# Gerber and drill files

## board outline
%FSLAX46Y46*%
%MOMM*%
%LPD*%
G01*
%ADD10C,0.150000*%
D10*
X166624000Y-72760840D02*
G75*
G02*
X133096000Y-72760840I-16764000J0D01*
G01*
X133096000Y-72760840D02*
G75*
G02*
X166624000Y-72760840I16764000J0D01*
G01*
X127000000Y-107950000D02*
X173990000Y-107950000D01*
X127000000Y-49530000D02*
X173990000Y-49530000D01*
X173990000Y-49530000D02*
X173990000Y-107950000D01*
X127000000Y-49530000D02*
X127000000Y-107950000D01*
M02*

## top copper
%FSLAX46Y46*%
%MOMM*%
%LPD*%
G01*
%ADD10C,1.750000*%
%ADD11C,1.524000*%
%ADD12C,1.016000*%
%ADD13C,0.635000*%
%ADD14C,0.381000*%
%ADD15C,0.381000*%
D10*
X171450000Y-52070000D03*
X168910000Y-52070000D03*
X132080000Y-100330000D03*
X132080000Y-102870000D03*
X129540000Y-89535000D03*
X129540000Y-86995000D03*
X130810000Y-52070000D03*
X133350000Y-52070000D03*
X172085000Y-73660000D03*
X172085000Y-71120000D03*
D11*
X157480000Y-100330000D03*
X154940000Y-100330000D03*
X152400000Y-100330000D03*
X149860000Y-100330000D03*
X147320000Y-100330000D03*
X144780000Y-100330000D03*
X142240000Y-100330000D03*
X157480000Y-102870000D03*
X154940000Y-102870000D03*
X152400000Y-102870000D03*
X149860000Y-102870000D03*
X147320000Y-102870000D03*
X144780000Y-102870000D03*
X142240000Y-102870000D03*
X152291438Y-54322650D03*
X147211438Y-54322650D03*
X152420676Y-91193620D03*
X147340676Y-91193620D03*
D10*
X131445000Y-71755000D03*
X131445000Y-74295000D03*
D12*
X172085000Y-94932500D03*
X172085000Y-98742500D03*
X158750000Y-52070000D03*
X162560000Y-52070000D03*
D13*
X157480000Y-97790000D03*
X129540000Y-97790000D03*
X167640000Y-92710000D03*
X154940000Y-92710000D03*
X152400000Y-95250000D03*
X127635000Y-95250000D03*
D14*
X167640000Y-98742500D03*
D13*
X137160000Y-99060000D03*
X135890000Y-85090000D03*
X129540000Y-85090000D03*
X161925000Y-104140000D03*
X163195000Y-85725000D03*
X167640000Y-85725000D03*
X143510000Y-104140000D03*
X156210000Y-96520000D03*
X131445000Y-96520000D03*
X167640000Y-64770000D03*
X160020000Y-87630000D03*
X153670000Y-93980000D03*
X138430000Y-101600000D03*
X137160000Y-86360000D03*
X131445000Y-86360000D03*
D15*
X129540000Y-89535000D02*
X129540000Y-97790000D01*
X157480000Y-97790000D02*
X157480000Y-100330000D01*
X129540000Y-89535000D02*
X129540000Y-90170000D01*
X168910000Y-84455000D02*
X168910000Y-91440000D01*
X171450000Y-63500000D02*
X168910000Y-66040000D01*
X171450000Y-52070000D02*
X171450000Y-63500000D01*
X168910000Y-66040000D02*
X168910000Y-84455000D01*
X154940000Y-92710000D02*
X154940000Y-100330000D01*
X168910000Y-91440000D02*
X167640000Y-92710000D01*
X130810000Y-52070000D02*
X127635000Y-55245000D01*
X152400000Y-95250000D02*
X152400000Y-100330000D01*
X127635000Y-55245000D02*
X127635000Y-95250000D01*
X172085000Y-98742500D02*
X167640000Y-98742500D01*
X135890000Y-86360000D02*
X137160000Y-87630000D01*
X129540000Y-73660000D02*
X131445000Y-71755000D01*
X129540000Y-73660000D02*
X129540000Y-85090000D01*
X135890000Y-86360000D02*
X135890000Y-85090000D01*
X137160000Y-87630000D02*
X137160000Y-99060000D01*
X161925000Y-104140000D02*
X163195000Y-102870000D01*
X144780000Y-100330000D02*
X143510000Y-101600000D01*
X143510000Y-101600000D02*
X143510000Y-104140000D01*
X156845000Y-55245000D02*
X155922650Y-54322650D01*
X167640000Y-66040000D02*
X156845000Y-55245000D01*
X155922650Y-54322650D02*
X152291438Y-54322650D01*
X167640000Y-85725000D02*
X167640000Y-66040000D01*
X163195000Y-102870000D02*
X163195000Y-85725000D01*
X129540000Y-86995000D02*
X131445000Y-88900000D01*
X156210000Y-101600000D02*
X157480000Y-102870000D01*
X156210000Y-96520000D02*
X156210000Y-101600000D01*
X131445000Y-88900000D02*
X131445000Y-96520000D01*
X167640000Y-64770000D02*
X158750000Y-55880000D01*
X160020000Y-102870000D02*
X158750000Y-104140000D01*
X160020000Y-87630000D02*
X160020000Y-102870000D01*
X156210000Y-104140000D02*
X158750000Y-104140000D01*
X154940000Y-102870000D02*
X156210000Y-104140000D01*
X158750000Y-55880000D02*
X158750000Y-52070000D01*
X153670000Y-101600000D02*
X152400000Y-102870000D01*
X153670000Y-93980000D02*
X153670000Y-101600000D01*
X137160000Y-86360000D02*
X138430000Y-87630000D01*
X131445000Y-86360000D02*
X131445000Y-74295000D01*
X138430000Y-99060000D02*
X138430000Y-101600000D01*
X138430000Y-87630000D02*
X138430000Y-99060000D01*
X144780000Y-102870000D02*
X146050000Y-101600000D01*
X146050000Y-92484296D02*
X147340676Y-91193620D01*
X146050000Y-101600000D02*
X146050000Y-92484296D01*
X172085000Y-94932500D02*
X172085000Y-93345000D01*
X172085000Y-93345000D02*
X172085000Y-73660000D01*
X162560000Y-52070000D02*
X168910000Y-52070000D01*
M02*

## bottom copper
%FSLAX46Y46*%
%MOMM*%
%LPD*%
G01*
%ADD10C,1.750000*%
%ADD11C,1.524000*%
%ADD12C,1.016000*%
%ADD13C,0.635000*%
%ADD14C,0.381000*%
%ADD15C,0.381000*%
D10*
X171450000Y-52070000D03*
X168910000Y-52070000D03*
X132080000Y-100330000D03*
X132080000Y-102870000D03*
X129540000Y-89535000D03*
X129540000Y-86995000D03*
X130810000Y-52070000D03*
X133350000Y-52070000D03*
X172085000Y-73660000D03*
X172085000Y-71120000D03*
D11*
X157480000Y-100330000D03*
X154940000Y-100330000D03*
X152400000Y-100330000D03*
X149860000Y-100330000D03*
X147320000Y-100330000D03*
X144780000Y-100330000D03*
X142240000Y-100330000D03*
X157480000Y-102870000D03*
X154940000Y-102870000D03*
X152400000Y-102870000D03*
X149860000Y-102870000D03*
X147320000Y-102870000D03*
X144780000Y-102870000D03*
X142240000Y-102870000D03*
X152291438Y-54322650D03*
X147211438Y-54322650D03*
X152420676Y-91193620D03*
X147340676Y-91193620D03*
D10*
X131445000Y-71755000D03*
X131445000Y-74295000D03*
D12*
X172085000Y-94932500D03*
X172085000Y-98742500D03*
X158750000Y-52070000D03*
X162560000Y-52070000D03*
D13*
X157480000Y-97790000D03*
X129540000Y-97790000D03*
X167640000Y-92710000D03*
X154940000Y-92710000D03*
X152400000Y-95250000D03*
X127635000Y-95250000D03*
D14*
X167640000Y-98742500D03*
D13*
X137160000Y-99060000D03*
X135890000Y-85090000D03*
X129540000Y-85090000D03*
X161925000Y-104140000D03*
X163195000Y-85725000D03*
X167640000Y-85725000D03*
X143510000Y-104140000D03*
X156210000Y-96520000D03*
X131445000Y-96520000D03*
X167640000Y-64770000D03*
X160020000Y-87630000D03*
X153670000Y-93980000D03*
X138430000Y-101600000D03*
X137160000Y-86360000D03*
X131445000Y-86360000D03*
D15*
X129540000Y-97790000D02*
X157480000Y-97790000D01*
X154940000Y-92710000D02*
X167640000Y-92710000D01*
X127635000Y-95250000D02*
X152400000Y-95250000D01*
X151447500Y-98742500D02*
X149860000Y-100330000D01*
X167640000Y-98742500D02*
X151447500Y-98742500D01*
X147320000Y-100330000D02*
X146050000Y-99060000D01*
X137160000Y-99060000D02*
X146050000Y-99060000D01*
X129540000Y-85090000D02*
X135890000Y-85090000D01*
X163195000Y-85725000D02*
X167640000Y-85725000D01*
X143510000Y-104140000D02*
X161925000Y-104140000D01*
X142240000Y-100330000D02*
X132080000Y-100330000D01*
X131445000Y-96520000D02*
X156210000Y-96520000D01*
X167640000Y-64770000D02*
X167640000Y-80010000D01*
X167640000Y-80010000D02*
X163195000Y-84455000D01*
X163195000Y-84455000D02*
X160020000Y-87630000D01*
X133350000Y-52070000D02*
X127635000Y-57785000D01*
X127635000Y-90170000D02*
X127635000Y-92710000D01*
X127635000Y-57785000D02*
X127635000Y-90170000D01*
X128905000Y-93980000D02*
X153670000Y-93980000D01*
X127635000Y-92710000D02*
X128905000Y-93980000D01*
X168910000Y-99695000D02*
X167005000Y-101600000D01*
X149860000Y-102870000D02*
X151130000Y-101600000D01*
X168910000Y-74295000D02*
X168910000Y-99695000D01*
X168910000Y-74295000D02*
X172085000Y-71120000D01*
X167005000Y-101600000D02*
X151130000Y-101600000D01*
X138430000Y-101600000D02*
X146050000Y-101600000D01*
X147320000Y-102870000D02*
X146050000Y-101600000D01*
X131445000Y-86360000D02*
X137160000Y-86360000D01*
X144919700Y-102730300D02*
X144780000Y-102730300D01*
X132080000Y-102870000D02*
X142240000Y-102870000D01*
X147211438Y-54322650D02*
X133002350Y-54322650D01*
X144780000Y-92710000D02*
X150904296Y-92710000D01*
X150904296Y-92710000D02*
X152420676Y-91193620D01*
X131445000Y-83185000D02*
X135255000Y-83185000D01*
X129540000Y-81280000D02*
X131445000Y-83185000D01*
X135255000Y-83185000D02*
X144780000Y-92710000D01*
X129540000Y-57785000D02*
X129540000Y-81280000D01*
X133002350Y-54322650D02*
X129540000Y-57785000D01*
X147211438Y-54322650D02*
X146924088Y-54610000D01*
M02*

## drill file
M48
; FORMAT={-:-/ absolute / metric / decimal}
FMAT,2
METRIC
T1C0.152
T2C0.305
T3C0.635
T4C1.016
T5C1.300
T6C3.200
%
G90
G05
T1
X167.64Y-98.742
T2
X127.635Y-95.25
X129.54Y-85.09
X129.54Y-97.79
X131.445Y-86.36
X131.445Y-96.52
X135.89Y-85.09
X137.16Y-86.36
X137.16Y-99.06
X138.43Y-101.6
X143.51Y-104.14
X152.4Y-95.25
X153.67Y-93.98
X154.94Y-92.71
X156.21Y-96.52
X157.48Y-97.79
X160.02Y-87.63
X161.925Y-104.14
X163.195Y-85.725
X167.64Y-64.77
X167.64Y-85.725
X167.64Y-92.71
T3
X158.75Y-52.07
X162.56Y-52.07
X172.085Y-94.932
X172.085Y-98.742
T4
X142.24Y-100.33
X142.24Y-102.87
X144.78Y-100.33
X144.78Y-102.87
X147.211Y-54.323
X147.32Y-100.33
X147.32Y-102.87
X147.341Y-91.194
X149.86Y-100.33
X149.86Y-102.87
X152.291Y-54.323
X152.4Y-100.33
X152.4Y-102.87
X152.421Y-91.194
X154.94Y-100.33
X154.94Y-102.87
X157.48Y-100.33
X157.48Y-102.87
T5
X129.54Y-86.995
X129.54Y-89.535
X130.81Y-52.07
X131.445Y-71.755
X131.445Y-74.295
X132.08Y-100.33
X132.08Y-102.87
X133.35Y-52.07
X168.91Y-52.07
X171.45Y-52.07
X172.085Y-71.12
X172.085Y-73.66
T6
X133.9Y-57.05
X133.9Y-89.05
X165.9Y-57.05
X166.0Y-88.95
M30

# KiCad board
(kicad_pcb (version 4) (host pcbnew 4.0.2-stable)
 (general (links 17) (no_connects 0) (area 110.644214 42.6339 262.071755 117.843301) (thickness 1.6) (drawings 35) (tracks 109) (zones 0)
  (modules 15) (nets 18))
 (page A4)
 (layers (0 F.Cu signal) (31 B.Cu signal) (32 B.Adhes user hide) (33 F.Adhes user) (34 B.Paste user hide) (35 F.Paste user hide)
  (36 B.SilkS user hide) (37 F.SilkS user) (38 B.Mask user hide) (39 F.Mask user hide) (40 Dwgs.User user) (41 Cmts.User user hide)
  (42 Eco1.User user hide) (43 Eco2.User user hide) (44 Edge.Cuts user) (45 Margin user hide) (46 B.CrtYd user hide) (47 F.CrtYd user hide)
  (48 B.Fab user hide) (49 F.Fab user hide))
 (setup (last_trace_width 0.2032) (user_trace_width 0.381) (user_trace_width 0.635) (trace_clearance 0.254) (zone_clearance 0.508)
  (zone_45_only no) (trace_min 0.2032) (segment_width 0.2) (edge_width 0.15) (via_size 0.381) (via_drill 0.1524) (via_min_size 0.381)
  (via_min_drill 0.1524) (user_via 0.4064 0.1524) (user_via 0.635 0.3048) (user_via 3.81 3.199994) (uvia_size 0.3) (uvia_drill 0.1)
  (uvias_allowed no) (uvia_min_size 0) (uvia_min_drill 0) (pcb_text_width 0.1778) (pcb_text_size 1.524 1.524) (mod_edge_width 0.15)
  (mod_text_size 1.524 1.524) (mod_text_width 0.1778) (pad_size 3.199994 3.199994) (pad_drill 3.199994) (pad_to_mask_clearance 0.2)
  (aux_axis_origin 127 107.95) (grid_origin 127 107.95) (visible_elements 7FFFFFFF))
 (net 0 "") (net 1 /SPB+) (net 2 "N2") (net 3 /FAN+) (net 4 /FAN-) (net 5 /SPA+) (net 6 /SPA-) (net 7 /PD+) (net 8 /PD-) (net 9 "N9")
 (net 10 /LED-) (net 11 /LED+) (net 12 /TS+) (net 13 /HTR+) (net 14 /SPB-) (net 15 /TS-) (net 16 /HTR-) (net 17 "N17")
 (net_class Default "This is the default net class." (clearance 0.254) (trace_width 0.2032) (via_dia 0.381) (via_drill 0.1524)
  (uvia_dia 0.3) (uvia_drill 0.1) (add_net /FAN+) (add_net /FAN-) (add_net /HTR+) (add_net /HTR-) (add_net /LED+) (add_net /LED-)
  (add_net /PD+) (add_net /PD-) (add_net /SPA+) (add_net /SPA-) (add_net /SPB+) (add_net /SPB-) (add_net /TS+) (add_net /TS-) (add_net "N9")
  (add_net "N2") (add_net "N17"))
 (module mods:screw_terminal (layer F.Cu) (at 170.18 52.07 180)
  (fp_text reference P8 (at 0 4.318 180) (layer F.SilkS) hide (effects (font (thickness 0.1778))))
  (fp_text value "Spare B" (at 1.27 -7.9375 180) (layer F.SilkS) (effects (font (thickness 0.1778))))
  (pad 1 thru_hole circle (at -1.27 0 180) (size 1.75 1.75) (drill 1.3) (layers *.Cu *.Mask F.SilkS) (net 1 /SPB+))
  (pad 2 thru_hole circle (at 1.27 0 180) (size 1.75 1.75) (drill 1.3) (layers *.Cu *.Mask F.SilkS) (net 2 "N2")))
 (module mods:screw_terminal (layer F.Cu) (at 132.08 101.6 270)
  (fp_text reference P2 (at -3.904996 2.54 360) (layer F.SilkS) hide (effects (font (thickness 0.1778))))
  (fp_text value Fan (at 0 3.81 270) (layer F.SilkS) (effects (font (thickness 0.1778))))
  (pad 1 thru_hole circle (at -1.27 0 270) (size 1.75 1.75) (drill 1.3) (layers *.Cu *.Mask F.SilkS) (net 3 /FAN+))
  (pad 2 thru_hole circle (at 1.27 0 270) (size 1.75 1.75) (drill 1.3) (layers *.Cu *.Mask F.SilkS) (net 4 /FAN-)))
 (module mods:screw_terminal (layer F.Cu) (at 129.54 88.265 90)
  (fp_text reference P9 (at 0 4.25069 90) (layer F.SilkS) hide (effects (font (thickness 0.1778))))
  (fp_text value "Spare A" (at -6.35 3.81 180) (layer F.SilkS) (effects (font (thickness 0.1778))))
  (pad 1 thru_hole circle (at -1.27 0 90) (size 1.75 1.75) (drill 1.3) (layers *.Cu *.Mask F.SilkS) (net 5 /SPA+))
  (pad 2 thru_hole circle (at 1.27 0 90) (size 1.75 1.75) (drill 1.3) (layers *.Cu *.Mask F.SilkS) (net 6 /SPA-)))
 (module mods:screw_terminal (layer F.Cu) (at 132.08 52.07)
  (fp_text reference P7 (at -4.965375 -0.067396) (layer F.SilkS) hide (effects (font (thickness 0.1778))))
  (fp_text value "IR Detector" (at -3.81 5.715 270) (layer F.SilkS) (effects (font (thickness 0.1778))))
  (pad 1 thru_hole circle (at -1.27 0) (size 1.75 1.75) (drill 1.3) (layers *.Cu *.Mask F.SilkS) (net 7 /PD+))
  (pad 2 thru_hole circle (at 1.27 0) (size 1.75 1.75) (drill 1.3) (layers *.Cu *.Mask F.SilkS) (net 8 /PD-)))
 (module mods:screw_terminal (layer F.Cu) (at 172.085 72.39 90)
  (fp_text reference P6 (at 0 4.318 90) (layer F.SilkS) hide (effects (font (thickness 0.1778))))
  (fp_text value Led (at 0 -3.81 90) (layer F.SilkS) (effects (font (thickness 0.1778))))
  (pad 1 thru_hole circle (at -1.27 0 90) (size 1.75 1.75) (drill 1.3) (layers *.Cu *.Mask F.SilkS) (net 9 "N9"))
  (pad 2 thru_hole circle (at 1.27 0 90) (size 1.75 1.75) (drill 1.3) (layers *.Cu *.Mask F.SilkS) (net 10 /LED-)))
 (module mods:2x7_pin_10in (layer F.Cu) (at 149.86 101.6 180)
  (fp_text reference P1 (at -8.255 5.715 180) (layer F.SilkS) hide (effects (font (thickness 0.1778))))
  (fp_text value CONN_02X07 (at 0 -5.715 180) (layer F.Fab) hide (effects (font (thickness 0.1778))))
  (pad 1 thru_hole circle (at -7.62 1.27 180) (size 1.524 1.524) (drill 1.016) (layers *.Cu *.Mask F.SilkS) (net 5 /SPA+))
  (pad 3 thru_hole circle (at -5.08 1.27 180) (size 1.524 1.524) (drill 1.016) (layers *.Cu *.Mask F.SilkS) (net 1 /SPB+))
  (pad 5 thru_hole circle (at -2.54 1.27 180) (size 1.524 1.524) (drill 1.016) (layers *.Cu *.Mask F.SilkS) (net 7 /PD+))
  (pad 7 thru_hole circle (at 0 1.27 180) (size 1.524 1.524) (drill 1.016) (layers *.Cu *.Mask F.SilkS) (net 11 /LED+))
  (pad 9 thru_hole circle (at 2.54 1.27 180) (size 1.524 1.524) (drill 1.016) (layers *.Cu *.Mask F.SilkS) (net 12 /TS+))
  (pad 11 thru_hole circle (at 5.08 1.27 180) (size 1.524 1.524) (drill 1.016) (layers *.Cu *.Mask F.SilkS) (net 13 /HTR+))
  (pad 13 thru_hole circle (at 7.62 1.27 180) (size 1.524 1.524) (drill 1.016) (layers *.Cu *.Mask F.SilkS) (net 3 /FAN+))
  (pad 2 thru_hole circle (at -7.62 -1.27 180) (size 1.524 1.524) (drill 1.016) (layers *.Cu *.Mask F.SilkS) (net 6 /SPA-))
  (pad 4 thru_hole circle (at -5.08 -1.27 180) (size 1.524 1.524) (drill 1.016) (layers *.Cu *.Mask F.SilkS) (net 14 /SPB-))
  (pad 6 thru_hole circle (at -2.54 -1.27 180) (size 1.524 1.524) (drill 1.016) (layers *.Cu *.Mask F.SilkS) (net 8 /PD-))
  (pad 8 thru_hole circle (at 0 -1.27 180) (size 1.524 1.524) (drill 1.016) (layers *.Cu *.Mask F.SilkS) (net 10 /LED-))
  (pad 10 thru_hole circle (at 2.54 -1.27 180) (size 1.524 1.524) (drill 1.016) (layers *.Cu *.Mask F.SilkS) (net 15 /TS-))
  (pad 12 thru_hole circle (at 5.08 -1.27 180) (size 1.524 1.524) (drill 1.016) (layers *.Cu *.Mask F.SilkS) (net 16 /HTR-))
  (pad 14 thru_hole circle (at 7.62 -1.27 180) (size 1.524 1.524) (drill 1.016) (layers *.Cu *.Mask F.SilkS) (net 4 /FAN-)))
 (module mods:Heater (layer F.Cu) (at 149.751438 54.32265 180)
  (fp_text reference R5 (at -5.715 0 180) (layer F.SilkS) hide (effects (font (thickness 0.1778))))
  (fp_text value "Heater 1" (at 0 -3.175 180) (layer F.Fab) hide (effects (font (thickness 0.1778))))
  (pad 1 thru_hole circle (at -2.54 0 180) (size 1.524 1.524) (drill 1.016) (layers *.Cu *.Mask F.SilkS) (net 13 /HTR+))
  (pad 2 thru_hole circle (at 2.54 0 180) (size 1.524 1.524) (drill 1.016) (layers *.Cu *.Mask F.SilkS) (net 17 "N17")))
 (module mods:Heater (layer F.Cu) (at 149.880676 91.19362 180)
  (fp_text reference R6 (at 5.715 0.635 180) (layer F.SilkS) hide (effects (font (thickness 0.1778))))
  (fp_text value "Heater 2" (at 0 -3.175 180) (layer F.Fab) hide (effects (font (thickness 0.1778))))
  (pad 1 thru_hole circle (at -2.54 0 180) (size 1.524 1.524) (drill 1.016) (layers *.Cu *.Mask F.SilkS) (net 17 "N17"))
  (pad 2 thru_hole circle (at 2.54 0 180) (size 1.524 1.524) (drill 1.016) (layers *.Cu *.Mask F.SilkS) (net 16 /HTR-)))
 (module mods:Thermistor (layer F.Cu) (at 131.445 73.025 270)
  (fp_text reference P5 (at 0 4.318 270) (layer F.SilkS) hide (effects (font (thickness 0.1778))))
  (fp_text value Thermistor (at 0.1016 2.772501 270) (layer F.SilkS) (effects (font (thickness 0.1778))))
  (pad 1 thru_hole circle (at -1.27 0 270) (size 1.75 1.75) (drill 1.3) (layers *.Cu *.Mask F.SilkS) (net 12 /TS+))
  (pad 2 thru_hole circle (at 1.27 0 270) (size 1.75 1.75) (drill 1.3) (layers *.Cu *.Mask F.SilkS) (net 15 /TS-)))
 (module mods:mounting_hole (layer F.Cu) (at 165.9 57.049924)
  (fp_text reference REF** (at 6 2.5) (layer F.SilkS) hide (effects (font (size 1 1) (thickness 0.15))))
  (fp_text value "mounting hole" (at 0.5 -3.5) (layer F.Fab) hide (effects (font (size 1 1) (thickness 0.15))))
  (pad "" np_thru_hole circle (at 0 0) (size 3.199994 3.199994) (drill 3.199994) (layers *.Cu *.Mask F.SilkS)))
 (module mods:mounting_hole (layer F.Cu) (at 133.899999 57.049924)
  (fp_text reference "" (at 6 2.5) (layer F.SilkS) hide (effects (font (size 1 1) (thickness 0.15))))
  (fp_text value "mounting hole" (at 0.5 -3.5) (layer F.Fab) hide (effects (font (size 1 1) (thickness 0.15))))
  (pad "" np_thru_hole circle (at 0 0) (size 3.199994 3.199994) (drill 3.199994) (layers *.Cu *.Mask F.SilkS)))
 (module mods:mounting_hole (layer F.Cu) (at 133.899999 89.04986)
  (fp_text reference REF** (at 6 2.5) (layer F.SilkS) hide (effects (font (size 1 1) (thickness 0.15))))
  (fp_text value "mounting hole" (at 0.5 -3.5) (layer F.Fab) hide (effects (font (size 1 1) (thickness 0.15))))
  (pad "" np_thru_hole circle (at 0 0) (size 3.199994 3.199994) (drill 3.199994) (layers *.Cu *.Mask F.SilkS)))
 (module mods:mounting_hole (layer F.Cu) (at 165.999998 88.950013)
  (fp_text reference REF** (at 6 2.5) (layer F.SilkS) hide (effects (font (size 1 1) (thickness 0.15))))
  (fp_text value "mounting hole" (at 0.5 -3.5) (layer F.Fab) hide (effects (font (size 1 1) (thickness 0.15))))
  (pad "" np_thru_hole circle (at 0 0) (size 3.199994 3.199994) (drill 3.199994) (layers *.Cu *.Mask F.SilkS)))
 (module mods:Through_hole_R (layer F.Cu) (at 172.085 96.8375 270)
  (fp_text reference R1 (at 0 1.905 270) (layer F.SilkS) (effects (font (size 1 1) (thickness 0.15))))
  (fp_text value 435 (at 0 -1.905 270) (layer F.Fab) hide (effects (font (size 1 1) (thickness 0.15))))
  (pad 2 thru_hole circle (at -1.905 0 270) (size 1.016 1.016) (drill 0.635) (layers *.Cu *.Mask F.SilkS) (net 9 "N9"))
  (pad 1 thru_hole circle (at 1.905 0 270) (size 1.016 1.016) (drill 0.635) (layers *.Cu *.Mask F.SilkS) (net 11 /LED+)))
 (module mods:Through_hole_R (layer F.Cu) (at 160.655 52.07)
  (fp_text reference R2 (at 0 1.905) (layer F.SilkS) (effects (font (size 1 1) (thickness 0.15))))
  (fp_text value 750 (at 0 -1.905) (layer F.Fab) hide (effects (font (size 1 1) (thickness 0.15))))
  (pad 2 thru_hole circle (at -1.905 0) (size 1.016 1.016) (drill 0.635) (layers *.Cu *.Mask F.SilkS) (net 14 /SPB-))
  (pad 1 thru_hole circle (at 1.905 0) (size 1.016 1.016) (drill 0.635) (layers *.Cu *.Mask F.SilkS) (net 2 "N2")))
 (gr_circle (center 149.86 72.76084) (end 133.096 72.76084) (layer Edge.Cuts) (width 0.15))
 (gr_line (start 127 107.95) (end 173.99 107.95) (angle 90) (layer Edge.Cuts) (width 0.15))
 (gr_line (start 127 49.53) (end 173.99 49.53) (angle 90) (layer Edge.Cuts) (width 0.15))
 (gr_line (start 173.99 49.53) (end 173.99 107.95) (angle 90) (layer Edge.Cuts) (width 0.15))
 (gr_line (start 127 49.53) (end 127 107.95) (angle 90) (layer Edge.Cuts) (width 0.15))
 (segment (start 129.54 89.535) (end 129.54 97.79) (width 0.381) (layer F.Cu) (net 5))
 (segment (start 157.48 97.79) (end 157.48 100.33) (width 0.381) (layer F.Cu) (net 5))
 (via (at 157.48 97.79) (size 0.635) (drill 0.3048) (layers F.Cu B.Cu) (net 5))
 (segment (start 129.54 97.79) (end 157.48 97.79) (width 0.381) (layer B.Cu) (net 5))
 (via (at 129.54 97.79) (size 0.635) (drill 0.3048) (layers F.Cu B.Cu) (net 5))
 (segment (start 129.54 89.535) (end 129.54 90.17) (width 0.381) (layer F.Cu) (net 5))
 (segment (start 168.91 84.455) (end 168.91 91.44) (width 0.381) (layer F.Cu) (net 1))
 (segment (start 171.45 63.5) (end 168.91 66.04) (width 0.381) (layer F.Cu) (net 1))
 (segment (start 171.45 52.07) (end 171.45 63.5) (width 0.381) (layer F.Cu) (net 1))
 (segment (start 168.91 66.04) (end 168.91 84.455) (width 0.381) (layer F.Cu) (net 1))
 (via (at 167.64 92.71) (size 0.635) (drill 0.3048) (layers F.Cu B.Cu) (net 1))
 (via (at 154.94 92.71) (size 0.635) (drill 0.3048) (layers F.Cu B.Cu) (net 1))
 (segment (start 154.94 92.71) (end 167.64 92.71) (width 0.381) (layer B.Cu) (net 1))
 (segment (start 154.94 92.71) (end 154.94 100.33) (width 0.381) (layer F.Cu) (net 1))
 (segment (start 168.91 91.44) (end 167.64 92.71) (width 0.381) (layer F.Cu) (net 1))
 (segment (start 130.81 52.07) (end 127.635 55.245) (width 0.381) (layer F.Cu) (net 7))
 (segment (start 152.4 95.25) (end 152.4 100.33) (width 0.381) (layer F.Cu) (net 7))
 (via (at 152.4 95.25) (size 0.635) (drill 0.3048) (layers F.Cu B.Cu) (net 7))
 (segment (start 127.635 95.25) (end 152.4 95.25) (width 0.381) (layer B.Cu) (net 7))
 (via (at 127.635 95.25) (size 0.635) (drill 0.3048) (layers F.Cu B.Cu) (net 7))
 (segment (start 127.635 55.245) (end 127.635 95.25) (width 0.381) (layer F.Cu) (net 7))
 (segment (start 172.085 98.7425) (end 167.64 98.7425) (width 0.381) (layer F.Cu) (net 11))
 (segment (start 151.4475 98.7425) (end 149.86 100.33) (width 0.381) (layer B.Cu) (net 11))
 (segment (start 167.64 98.7425) (end 151.4475 98.7425) (width 0.381) (layer B.Cu) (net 11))
 (via (at 167.64 98.7425) (size 0.381) (drill 0.1524) (layers F.Cu B.Cu) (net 11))
 (segment (start 135.89 86.36) (end 137.16 87.63) (width 0.381) (layer F.Cu) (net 12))
 (via (at 137.16 99.06) (size 0.635) (drill 0.3048) (layers F.Cu B.Cu) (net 12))
 (segment (start 147.32 100.33) (end 146.05 99.06) (width 0.381) (layer B.Cu) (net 12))
 (segment (start 137.16 99.06) (end 146.05 99.06) (width 0.381) (layer B.Cu) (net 12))
 (segment (start 129.54 73.66) (end 131.445 71.755) (width 0.381) (layer F.Cu) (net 12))
 (via (at 135.89 85.09) (size 0.635) (drill 0.3048) (layers F.Cu B.Cu) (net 12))
 (segment (start 129.54 85.09) (end 135.89 85.09) (width 0.381) (layer B.Cu) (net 12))
 (via (at 129.54 85.09) (size 0.635) (drill 0.3048) (layers F.Cu B.Cu) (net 12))
 (segment (start 129.54 73.66) (end 129.54 85.09) (width 0.381) (layer F.Cu) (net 12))
 (segment (start 135.89 86.36) (end 135.89 85.09) (width 0.381) (layer F.Cu) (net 12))
 (segment (start 137.16 87.63) (end 137.16 99.06) (width 0.381) (layer F.Cu) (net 12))
 (segment (start 161.925 104.14) (end 163.195 102.87) (width 0.381) (layer F.Cu) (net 13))
 (via (at 161.925 104.14) (size 0.635) (drill 0.3048) (layers F.Cu B.Cu) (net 13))
 (via (at 163.195 85.725) (size 0.635) (drill 0.3048) (layers F.Cu B.Cu) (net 13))
 (segment (start 163.195 85.725) (end 167.64 85.725) (width 0.381) (layer B.Cu) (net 13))
 (via (at 167.64 85.725) (size 0.635) (drill 0.3048) (layers F.Cu B.Cu) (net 13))
 (segment (start 144.78 100.33) (end 143.51 101.6) (width 0.381) (layer F.Cu) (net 13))
 (via (at 143.51 104.14) (size 0.635) (drill 0.3048) (layers F.Cu B.Cu) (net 13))
 (segment (start 143.51 101.6) (end 143.51 104.14) (width 0.381) (layer F.Cu) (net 13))
 (segment (start 143.51 104.14) (end 161.925 104.14) (width 0.381) (layer B.Cu) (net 13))
 (segment (start 156.845 55.245) (end 155.92265 54.32265) (width 0.381) (layer F.Cu) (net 13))
 (segment (start 167.64 66.04) (end 156.845 55.245) (width 0.381) (layer F.Cu) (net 13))
 (segment (start 155.92265 54.32265) (end 152.291438 54.32265) (width 0.381) (layer F.Cu) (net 13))
 (segment (start 167.64 85.725) (end 167.64 66.04) (width 0.381) (layer F.Cu) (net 13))
 (segment (start 163.195 102.87) (end 163.195 85.725) (width 0.381) (layer F.Cu) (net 13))
 (segment (start 142.24 100.33) (end 132.08 100.33) (width 0.381) (layer B.Cu) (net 3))
 (segment (start 129.54 86.995) (end 131.445 88.9) (width 0.381) (layer F.Cu) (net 6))
 (segment (start 156.21 101.6) (end 157.48 102.87) (width 0.381) (layer F.Cu) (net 6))
 (segment (start 156.21 96.52) (end 156.21 101.6) (width 0.381) (layer F.Cu) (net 6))
 (via (at 156.21 96.52) (size 0.635) (drill 0.3048) (layers F.Cu B.Cu) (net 6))
 (segment (start 131.445 96.52) (end 156.21 96.52) (width 0.381) (layer B.Cu) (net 6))
 (via (at 131.445 96.52) (size 0.635) (drill 0.3048) (layers F.Cu B.Cu) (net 6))
 (segment (start 131.445 88.9) (end 131.445 96.52) (width 0.381) (layer F.Cu) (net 6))
 (segment (start 167.64 64.77) (end 158.75 55.88) (width 0.381) (layer F.Cu) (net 14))
 (via (at 167.64 64.77) (size 0.635) (drill 0.3048) (layers F.Cu B.Cu) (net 14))
 (segment (start 167.64 64.77) (end 167.64 80.01) (width 0.381) (layer B.Cu) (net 14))
 (segment (start 167.64 80.01) (end 163.195 84.455) (width 0.381) (layer B.Cu) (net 14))
 (segment (start 160.02 102.87) (end 158.75 104.14) (width 0.381) (layer F.Cu) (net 14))
 (segment (start 160.02 87.63) (end 160.02 102.87) (width 0.381) (layer F.Cu) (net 14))
 (via (at 160.02 87.63) (size 0.635) (drill 0.3048) (layers F.Cu B.Cu) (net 14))
 (segment (start 163.195 84.455) (end 160.02 87.63) (width 0.381) (layer B.Cu) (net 14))
 (segment (start 156.21 104.14) (end 158.75 104.14) (width 0.381) (layer F.Cu) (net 14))
 (segment (start 154.94 102.87) (end 156.21 104.14) (width 0.381) (layer F.Cu) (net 14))
 (segment (start 158.75 55.88) (end 158.75 52.07) (width 0.381) (layer F.Cu) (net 14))
 (segment (start 133.35 52.07) (end 127.635 57.785) (width 0.381) (layer B.Cu) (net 8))
 (segment (start 127.635 90.17) (end 127.635 92.71) (width 0.381) (layer B.Cu) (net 8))
 (segment (start 127.635 57.785) (end 127.635 90.17) (width 0.381) (layer B.Cu) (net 8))
 (segment (start 153.67 101.6) (end 152.4 102.87) (width 0.381) (layer F.Cu) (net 8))
 (segment (start 153.67 93.98) (end 153.67 101.6) (width 0.381) (layer F.Cu) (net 8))
 (via (at 153.67 93.98) (size 0.635) (drill 0.3048) (layers F.Cu B.Cu) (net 8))
 (segment (start 128.905 93.98) (end 153.67 93.98) (width 0.381) (layer B.Cu) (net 8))
 (segment (start 127.635 92.71) (end 128.905 93.98) (width 0.381) (layer B.Cu) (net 8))
 (segment (start 168.91 99.695) (end 167.005 101.6) (width 0.381) (layer B.Cu) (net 10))
 (segment (start 149.86 102.87) (end 151.13 101.6) (width 0.381) (layer B.Cu) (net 10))
 (segment (start 168.91 74.295) (end 168.91 99.695) (width 0.381) (layer B.Cu) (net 10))
 (segment (start 168.91 74.295) (end 172.085 71.12) (width 0.381) (layer B.Cu) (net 10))
 (segment (start 167.005 101.6) (end 151.13 101.6) (width 0.381) (layer B.Cu) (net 10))
 (segment (start 137.16 86.36) (end 138.43 87.63) (width 0.381) (layer F.Cu) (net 15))
 (via (at 138.43 101.6) (size 0.635) (drill 0.3048) (layers F.Cu B.Cu) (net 15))
 (segment (start 138.43 101.6) (end 146.05 101.6) (width 0.381) (layer B.Cu) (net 15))
 (segment (start 147.32 102.87) (end 146.05 101.6) (width 0.381) (layer B.Cu) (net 15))
 (segment (start 131.445 86.36) (end 131.445 74.295) (width 0.381) (layer F.Cu) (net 15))
 (via (at 137.16 86.36) (size 0.635) (drill 0.3048) (layers F.Cu B.Cu) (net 15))
 (segment (start 131.445 86.36) (end 137.16 86.36) (width 0.381) (layer B.Cu) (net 15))
 (via (at 131.445 86.36) (size 0.635) (drill 0.3048) (layers F.Cu B.Cu) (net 15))
 (segment (start 138.43 99.06) (end 138.43 101.6) (width 0.381) (layer F.Cu) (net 15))
 (segment (start 138.43 87.63) (end 138.43 99.06) (width 0.381) (layer F.Cu) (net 15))
 (segment (start 144.78 102.87) (end 146.05 101.6) (width 0.381) (layer F.Cu) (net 16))
 (segment (start 146.05 92.484296) (end 147.340676 91.19362) (width 0.381) (layer F.Cu) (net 16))
 (segment (start 146.05 101.6) (end 146.05 92.484296) (width 0.381) (layer F.Cu) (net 16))
 (segment (start 144.9197 102.7303) (end 144.78 102.7303) (width 0.381) (layer B.Cu) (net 16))
 (segment (start 132.08 102.87) (end 142.24 102.87) (width 0.381) (layer B.Cu) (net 4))
 (segment (start 172.085 94.9325) (end 172.085 93.345) (width 0.381) (layer F.Cu) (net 9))
 (segment (start 172.085 93.345) (end 172.085 73.66) (width 0.381) (layer F.Cu) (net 9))
 (segment (start 162.56 52.07) (end 168.91 52.07) (width 0.381) (layer F.Cu) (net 2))
 (segment (start 147.211438 54.32265) (end 133.00235 54.32265) (width 0.381) (layer B.Cu) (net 17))
 (segment (start 144.78 92.71) (end 150.904296 92.71) (width 0.381) (layer B.Cu) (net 17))
 (segment (start 150.904296 92.71) (end 152.420676 91.19362) (width 0.381) (layer B.Cu) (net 17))
 (segment (start 131.445 83.185) (end 135.255 83.185) (width 0.381) (layer B.Cu) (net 17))
 (segment (start 129.54 81.28) (end 131.445 83.185) (width 0.381) (layer B.Cu) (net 17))
 (segment (start 135.255 83.185) (end 144.78 92.71) (width 0.381) (layer B.Cu) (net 17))
 (segment (start 129.54 57.785) (end 129.54 81.28) (width 0.381) (layer B.Cu) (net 17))
 (segment (start 133.00235 54.32265) (end 129.54 57.785) (width 0.381) (layer B.Cu) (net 17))
 (segment (start 147.211438 54.32265) (end 146.924088 54.61) (width 0.381) (layer B.Cu) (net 17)))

